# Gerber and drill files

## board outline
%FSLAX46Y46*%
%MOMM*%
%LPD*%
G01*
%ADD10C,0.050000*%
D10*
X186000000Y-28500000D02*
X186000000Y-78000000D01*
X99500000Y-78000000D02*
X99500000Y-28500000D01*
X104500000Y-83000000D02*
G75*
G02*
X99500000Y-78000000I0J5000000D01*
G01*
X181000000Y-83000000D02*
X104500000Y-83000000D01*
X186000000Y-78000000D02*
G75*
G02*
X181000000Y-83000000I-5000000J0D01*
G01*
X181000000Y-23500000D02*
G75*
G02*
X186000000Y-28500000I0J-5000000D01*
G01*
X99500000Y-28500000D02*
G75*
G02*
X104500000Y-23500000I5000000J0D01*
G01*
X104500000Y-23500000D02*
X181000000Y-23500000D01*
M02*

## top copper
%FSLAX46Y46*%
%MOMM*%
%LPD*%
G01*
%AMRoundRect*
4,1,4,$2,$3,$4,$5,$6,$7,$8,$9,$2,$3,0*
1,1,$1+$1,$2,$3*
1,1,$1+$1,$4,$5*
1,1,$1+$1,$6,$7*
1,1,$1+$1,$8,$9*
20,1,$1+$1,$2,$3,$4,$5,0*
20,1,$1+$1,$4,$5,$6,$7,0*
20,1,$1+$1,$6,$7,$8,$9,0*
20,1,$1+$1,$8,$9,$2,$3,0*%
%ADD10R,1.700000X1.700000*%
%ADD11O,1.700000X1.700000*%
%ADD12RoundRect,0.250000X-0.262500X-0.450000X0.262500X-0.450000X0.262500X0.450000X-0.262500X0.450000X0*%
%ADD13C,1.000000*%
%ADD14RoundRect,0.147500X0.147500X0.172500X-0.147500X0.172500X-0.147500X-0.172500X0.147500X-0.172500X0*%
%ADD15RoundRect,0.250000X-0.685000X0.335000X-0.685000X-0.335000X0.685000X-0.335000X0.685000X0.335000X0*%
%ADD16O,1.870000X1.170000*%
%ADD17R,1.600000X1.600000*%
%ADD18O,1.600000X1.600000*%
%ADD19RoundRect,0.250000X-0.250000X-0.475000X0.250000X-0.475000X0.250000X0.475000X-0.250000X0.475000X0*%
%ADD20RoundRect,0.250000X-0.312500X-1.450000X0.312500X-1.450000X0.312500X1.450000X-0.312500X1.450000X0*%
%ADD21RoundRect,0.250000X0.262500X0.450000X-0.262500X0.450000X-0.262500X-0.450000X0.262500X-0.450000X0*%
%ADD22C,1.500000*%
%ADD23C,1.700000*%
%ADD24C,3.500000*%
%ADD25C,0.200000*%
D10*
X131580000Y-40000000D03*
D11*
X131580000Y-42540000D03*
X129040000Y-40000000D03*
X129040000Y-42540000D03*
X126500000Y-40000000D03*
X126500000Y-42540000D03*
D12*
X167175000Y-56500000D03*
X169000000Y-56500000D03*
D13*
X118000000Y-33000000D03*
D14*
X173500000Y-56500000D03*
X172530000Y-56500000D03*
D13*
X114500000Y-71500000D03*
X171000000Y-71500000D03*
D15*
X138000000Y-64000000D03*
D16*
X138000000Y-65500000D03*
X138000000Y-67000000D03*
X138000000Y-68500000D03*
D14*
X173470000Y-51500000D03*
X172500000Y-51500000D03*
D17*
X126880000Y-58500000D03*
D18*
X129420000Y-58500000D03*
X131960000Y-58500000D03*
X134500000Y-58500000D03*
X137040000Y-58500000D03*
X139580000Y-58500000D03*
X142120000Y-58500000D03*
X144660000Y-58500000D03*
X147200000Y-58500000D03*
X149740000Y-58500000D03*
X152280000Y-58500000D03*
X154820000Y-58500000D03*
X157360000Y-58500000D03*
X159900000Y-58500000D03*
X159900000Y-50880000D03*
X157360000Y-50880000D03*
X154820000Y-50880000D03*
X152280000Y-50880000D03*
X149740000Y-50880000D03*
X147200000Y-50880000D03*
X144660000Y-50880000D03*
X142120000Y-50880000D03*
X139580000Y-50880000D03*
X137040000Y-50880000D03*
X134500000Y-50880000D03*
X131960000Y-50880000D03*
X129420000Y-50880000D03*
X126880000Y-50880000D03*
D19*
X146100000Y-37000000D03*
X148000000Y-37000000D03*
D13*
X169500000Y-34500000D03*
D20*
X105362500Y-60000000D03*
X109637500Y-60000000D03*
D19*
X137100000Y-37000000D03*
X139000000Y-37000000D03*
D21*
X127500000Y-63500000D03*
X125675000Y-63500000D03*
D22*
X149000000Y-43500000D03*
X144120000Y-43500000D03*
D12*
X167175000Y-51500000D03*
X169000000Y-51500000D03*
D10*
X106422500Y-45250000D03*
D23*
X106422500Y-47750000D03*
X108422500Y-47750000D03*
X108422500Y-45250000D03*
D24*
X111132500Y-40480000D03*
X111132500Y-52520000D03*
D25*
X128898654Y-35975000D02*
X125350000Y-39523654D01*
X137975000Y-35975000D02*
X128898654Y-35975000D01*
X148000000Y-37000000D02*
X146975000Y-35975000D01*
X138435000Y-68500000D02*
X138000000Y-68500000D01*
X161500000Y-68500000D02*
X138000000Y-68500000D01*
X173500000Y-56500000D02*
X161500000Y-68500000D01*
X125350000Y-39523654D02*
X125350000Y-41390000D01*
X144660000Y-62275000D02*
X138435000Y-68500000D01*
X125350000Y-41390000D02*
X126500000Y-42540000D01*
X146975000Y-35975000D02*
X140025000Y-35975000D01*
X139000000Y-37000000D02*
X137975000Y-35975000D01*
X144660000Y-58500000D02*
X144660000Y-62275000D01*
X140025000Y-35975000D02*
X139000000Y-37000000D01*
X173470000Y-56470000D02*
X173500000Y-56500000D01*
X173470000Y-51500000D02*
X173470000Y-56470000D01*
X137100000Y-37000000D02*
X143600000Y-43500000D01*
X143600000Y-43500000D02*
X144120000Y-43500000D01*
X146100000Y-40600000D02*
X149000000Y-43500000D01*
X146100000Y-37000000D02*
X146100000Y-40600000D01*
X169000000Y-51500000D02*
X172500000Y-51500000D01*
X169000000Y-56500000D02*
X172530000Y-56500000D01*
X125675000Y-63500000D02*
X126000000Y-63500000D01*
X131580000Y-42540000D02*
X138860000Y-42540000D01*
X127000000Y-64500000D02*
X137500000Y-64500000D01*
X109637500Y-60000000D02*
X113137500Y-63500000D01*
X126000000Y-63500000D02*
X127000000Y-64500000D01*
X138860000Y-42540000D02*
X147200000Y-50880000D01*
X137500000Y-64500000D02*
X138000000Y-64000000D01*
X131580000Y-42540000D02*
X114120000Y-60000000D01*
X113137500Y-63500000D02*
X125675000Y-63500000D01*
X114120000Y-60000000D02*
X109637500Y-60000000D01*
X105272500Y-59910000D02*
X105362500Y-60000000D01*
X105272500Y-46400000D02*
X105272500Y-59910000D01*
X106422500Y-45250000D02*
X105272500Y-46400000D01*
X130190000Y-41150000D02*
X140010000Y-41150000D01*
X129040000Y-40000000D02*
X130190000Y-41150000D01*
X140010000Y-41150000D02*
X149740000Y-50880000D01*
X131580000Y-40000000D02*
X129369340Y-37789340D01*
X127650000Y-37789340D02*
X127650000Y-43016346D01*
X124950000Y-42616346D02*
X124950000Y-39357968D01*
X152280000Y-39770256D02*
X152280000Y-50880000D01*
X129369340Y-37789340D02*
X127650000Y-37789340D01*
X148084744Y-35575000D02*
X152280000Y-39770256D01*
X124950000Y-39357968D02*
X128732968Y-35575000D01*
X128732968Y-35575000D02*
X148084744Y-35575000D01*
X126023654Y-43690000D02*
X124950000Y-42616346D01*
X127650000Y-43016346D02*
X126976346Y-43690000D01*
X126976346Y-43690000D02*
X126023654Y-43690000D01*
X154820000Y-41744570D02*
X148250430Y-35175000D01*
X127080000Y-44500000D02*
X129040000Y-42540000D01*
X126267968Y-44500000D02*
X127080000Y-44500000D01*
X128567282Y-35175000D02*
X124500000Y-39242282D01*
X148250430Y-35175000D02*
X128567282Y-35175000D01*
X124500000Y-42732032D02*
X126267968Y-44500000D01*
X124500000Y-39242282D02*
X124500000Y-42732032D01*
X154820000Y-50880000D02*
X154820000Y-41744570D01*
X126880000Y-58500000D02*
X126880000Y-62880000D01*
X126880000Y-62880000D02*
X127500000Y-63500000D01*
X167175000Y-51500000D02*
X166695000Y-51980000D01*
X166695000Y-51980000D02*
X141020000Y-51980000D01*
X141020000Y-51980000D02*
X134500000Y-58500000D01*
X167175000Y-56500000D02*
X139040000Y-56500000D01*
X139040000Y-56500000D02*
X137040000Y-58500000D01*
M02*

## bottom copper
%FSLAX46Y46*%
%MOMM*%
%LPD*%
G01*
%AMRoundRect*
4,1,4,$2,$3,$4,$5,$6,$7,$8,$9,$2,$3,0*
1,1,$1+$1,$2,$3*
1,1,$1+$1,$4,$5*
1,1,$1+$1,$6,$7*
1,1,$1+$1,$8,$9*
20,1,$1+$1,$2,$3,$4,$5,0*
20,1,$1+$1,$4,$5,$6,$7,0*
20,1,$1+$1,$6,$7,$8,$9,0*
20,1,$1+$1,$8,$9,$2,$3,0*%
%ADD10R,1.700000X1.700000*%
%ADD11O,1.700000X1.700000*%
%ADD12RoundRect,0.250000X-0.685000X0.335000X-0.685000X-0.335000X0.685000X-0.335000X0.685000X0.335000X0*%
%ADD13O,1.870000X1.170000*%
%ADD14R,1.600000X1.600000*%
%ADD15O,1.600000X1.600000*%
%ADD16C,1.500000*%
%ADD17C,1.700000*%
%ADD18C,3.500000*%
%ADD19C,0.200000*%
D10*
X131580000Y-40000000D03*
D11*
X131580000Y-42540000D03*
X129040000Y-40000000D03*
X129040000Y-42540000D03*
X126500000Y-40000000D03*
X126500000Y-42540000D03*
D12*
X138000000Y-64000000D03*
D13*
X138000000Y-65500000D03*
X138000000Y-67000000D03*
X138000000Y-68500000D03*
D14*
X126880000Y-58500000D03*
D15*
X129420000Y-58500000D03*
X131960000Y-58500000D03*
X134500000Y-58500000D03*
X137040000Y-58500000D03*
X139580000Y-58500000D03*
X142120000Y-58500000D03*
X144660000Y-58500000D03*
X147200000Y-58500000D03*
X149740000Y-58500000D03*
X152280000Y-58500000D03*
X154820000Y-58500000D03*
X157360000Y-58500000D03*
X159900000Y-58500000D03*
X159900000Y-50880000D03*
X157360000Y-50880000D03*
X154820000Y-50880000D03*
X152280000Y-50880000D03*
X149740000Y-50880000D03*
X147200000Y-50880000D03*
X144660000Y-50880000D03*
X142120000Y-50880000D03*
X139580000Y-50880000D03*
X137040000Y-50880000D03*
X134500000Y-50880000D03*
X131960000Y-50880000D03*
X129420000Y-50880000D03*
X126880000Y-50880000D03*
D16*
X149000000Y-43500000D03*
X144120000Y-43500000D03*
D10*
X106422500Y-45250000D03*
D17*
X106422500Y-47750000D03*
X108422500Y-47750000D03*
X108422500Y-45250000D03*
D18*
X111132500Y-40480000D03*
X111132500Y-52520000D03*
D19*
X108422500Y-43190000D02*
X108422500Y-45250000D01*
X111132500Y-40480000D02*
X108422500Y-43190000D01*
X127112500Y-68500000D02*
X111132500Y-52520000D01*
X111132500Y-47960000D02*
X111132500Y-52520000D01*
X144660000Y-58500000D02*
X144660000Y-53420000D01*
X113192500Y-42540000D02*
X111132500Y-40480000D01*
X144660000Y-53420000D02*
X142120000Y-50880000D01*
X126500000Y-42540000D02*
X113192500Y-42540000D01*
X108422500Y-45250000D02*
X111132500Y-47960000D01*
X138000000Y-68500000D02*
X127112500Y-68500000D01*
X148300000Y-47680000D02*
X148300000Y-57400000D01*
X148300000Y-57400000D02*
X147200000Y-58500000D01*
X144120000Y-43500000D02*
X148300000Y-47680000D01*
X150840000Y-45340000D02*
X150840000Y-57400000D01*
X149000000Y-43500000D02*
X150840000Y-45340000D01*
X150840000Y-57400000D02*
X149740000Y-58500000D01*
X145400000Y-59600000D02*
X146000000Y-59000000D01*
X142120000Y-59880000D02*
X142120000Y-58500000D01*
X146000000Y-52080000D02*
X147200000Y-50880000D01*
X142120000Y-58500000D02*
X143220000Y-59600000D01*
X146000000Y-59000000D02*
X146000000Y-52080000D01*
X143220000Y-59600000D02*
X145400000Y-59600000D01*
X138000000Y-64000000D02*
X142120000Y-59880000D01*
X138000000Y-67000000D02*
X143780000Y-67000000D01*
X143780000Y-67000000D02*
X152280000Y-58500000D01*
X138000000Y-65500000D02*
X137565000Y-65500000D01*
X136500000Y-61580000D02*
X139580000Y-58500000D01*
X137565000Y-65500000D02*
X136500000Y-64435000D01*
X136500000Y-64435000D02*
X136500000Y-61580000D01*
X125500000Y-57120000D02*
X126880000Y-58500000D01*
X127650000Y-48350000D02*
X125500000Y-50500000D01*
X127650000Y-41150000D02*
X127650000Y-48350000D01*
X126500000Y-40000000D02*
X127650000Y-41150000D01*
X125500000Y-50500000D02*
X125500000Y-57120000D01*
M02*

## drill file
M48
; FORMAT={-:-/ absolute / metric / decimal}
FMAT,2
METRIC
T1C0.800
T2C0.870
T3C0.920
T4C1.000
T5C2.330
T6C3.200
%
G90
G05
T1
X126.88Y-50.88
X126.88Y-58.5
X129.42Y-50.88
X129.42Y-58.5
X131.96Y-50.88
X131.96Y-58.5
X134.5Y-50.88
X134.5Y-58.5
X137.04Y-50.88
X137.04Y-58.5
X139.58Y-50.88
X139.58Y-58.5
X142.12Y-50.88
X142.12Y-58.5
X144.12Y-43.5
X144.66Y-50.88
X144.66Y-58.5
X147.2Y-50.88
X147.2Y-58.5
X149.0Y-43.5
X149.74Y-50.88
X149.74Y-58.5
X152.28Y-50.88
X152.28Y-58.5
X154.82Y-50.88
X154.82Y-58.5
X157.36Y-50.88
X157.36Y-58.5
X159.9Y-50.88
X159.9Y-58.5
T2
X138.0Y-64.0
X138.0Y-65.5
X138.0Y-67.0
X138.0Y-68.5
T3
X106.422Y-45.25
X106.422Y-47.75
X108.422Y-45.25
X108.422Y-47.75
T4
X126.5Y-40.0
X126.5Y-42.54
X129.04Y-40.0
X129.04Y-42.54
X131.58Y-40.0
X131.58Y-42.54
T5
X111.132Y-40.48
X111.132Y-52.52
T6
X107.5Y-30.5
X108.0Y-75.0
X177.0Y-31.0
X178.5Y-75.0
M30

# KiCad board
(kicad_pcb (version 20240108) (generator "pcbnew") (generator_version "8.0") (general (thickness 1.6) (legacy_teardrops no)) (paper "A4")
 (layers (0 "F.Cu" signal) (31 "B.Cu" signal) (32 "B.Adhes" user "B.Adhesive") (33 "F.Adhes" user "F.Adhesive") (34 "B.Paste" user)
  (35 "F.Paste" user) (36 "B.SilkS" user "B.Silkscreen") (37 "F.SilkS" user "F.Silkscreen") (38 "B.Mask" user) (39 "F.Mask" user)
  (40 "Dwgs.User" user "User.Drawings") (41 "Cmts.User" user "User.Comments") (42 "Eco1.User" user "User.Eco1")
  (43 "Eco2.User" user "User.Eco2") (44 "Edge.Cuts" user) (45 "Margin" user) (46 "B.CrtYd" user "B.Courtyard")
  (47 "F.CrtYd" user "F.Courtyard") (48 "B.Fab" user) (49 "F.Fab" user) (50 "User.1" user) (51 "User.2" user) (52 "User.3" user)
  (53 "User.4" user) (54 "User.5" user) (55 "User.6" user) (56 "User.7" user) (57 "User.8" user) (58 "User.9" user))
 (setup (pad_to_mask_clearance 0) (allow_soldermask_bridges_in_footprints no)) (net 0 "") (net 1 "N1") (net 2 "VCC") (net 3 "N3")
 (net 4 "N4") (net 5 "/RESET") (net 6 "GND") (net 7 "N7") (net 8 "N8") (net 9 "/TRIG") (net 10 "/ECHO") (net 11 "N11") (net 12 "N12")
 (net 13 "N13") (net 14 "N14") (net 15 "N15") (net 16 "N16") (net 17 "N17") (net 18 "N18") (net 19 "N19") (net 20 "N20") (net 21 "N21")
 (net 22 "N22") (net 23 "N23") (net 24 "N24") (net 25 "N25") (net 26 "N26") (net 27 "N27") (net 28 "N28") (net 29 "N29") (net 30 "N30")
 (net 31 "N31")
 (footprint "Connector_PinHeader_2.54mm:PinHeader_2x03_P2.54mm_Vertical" (layer "F.Cu") (at 131.58 40 -90)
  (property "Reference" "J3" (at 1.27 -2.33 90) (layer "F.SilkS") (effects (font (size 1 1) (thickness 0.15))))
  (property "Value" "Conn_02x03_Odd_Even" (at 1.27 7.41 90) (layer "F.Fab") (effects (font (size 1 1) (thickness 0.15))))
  (pad "1" thru_hole rect (at 0 0 270) (size 1.7 1.7) (drill 1) (layers "*.Cu" "*.Mask") (remove_unused_layers no) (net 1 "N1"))
  (pad "2" thru_hole oval (at 2.54 0 270) (size 1.7 1.7) (drill 1) (layers "*.Cu" "*.Mask") (remove_unused_layers no) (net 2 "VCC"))
  (pad "3" thru_hole oval (at 0 2.54 270) (size 1.7 1.7) (drill 1) (layers "*.Cu" "*.Mask") (remove_unused_layers no) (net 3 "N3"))
  (pad "4" thru_hole oval (at 2.54 2.54 270) (size 1.7 1.7) (drill 1) (layers "*.Cu" "*.Mask") (remove_unused_layers no) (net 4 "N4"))
  (pad "5" thru_hole oval (at 0 5.08 270) (size 1.7 1.7) (drill 1) (layers "*.Cu" "*.Mask") (remove_unused_layers no) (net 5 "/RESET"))
  (pad "6" thru_hole oval (at 2.54 5.08 270) (size 1.7 1.7) (drill 1) (layers "*.Cu" "*.Mask") (remove_unused_layers no) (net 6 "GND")))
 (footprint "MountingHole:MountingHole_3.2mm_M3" (layer "F.Cu") (at 108 75)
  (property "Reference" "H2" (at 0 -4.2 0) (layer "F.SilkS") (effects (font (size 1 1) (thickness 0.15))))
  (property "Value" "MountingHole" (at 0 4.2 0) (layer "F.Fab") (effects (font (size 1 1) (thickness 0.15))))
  (pad "" np_thru_hole circle (at 0 0) (size 3.2 3.2) (drill 3.2) (layers "*.Cu" "*.Mask")))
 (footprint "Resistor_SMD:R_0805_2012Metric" (layer "F.Cu") (at 168.0875 56.5)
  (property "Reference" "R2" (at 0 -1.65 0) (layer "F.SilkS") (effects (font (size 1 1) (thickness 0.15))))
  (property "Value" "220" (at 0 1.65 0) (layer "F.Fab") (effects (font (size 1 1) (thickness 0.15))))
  (pad "1" smd roundrect (at -0.9125 0) (size 1.025 1.4) (layers "F.Cu" "F.Paste" "F.Mask") (roundrect_rratio 0.243902) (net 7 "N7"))
  (pad "2" smd roundrect (at 0.9125 0) (size 1.025 1.4) (layers "F.Cu" "F.Paste" "F.Mask") (roundrect_rratio 0.243902) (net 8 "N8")))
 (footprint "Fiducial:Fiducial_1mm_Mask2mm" (layer "F.Cu") (at 118 33)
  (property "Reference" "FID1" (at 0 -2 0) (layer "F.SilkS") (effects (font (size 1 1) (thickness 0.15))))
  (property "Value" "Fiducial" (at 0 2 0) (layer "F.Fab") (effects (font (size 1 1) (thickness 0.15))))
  (pad "" smd circle (at 0 0) (size 1 1) (layers "F.Cu" "F.Mask") (solder_mask_margin 0.5) (clearance 0.5)))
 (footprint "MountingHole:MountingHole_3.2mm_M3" (layer "F.Cu") (at 177 31)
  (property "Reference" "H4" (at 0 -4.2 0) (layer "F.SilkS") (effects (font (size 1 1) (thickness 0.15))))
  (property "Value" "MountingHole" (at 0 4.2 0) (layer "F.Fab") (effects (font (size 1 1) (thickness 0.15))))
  (pad "" np_thru_hole circle (at 0 0) (size 3.2 3.2) (drill 3.2) (layers "*.Cu" "*.Mask")))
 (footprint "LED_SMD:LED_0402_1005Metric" (layer "F.Cu") (at 173.015 56.5 180)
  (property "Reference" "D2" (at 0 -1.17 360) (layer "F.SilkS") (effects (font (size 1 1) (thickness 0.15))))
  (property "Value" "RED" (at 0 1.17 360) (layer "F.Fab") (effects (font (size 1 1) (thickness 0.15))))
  (pad "1" smd roundrect (at -0.485 0 180) (size 0.59 0.64) (layers "F.Cu" "F.Paste" "F.Mask") (roundrect_rratio 0.25) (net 6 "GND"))
  (pad "2" smd roundrect (at 0.485 0 180) (size 0.59 0.64) (layers "F.Cu" "F.Paste" "F.Mask") (roundrect_rratio 0.25) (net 8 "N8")))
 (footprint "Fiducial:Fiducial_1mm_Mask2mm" (layer "F.Cu") (at 114.5 71.5)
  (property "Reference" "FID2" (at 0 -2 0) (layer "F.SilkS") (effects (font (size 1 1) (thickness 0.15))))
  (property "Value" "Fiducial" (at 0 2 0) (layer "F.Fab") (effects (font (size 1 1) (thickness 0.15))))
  (pad "" smd circle (at 0 0) (size 1 1) (layers "F.Cu" "F.Mask") (solder_mask_margin 0.5) (clearance 0.5)))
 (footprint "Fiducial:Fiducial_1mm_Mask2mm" (layer "F.Cu") (at 171 71.5)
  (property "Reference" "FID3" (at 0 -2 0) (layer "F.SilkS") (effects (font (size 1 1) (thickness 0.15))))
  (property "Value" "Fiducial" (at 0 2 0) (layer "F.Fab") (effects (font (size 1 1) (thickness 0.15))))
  (pad "" smd circle (at 0 0) (size 1 1) (layers "F.Cu" "F.Mask") (solder_mask_margin 0.5) (clearance 0.5)))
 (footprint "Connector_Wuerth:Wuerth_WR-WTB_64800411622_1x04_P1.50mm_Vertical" (layer "F.Cu") (at 138 64 -90)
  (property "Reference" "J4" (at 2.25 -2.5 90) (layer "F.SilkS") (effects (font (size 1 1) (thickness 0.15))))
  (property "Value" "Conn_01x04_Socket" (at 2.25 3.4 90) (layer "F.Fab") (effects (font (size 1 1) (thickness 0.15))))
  (pad "1" thru_hole roundrect (at 0 0 270) (size 1.17 1.87) (drill 0.87) (layers "*.Cu" "*.Mask") (remove_unused_layers no)
   (roundrect_rratio 0.213675) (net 2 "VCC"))
  (pad "2" thru_hole oval (at 1.5 0 270) (size 1.17 1.87) (drill 0.87) (layers "*.Cu" "*.Mask") (remove_unused_layers no) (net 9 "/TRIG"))
  (pad "3" thru_hole oval (at 3 0 270) (size 1.17 1.87) (drill 0.87) (layers "*.Cu" "*.Mask") (remove_unused_layers no) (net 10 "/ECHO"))
  (pad "4" thru_hole oval (at 4.5 0 270) (size 1.17 1.87) (drill 0.87) (layers "*.Cu" "*.Mask") (remove_unused_layers no) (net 6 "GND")))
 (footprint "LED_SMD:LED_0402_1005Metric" (layer "F.Cu") (at 172.985 51.5 180)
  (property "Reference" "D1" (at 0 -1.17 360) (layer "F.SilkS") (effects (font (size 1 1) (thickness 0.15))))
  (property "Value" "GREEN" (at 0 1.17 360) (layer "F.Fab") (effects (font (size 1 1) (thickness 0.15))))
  (pad "1" smd roundrect (at -0.485 0 180) (size 0.59 0.64) (layers "F.Cu" "F.Paste" "F.Mask") (roundrect_rratio 0.25) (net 6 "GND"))
  (pad "2" smd roundrect (at 0.485 0 180) (size 0.59 0.64) (layers "F.Cu" "F.Paste" "F.Mask") (roundrect_rratio 0.25) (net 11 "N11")))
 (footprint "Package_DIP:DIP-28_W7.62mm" (layer "F.Cu") (at 126.88 58.5 90)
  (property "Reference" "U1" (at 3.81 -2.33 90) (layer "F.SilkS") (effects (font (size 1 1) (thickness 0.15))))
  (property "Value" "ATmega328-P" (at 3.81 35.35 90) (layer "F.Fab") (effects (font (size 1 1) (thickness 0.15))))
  (pad "1" thru_hole rect (at 0 0 90) (size 1.6 1.6) (drill 0.8) (layers "*.Cu" "*.Mask") (remove_unused_layers no) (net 5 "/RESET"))
  (pad "2" thru_hole oval (at 0 2.54 90) (size 1.6 1.6) (drill 0.8) (layers "*.Cu" "*.Mask") (remove_unused_layers no) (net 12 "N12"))
  (pad "3" thru_hole oval (at 0 5.08 90) (size 1.6 1.6) (drill 0.8) (layers "*.Cu" "*.Mask") (remove_unused_layers no) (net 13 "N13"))
  (pad "4" thru_hole oval (at 0 7.62 90) (size 1.6 1.6) (drill 0.8) (layers "*.Cu" "*.Mask") (remove_unused_layers no) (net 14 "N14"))
  (pad "5" thru_hole oval (at 0 10.16 90) (size 1.6 1.6) (drill 0.8) (layers "*.Cu" "*.Mask") (remove_unused_layers no) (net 7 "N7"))
  (pad "6" thru_hole oval (at 0 12.7 90) (size 1.6 1.6) (drill 0.8) (layers "*.Cu" "*.Mask") (remove_unused_layers no) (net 9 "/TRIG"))
  (pad "7" thru_hole oval (at 0 15.24 90) (size 1.6 1.6) (drill 0.8) (layers "*.Cu" "*.Mask") (remove_unused_layers no) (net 2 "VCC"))
  (pad "8" thru_hole oval (at 0 17.78 90) (size 1.6 1.6) (drill 0.8) (layers "*.Cu" "*.Mask") (remove_unused_layers no) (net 6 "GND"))
  (pad "9" thru_hole oval (at 0 20.32 90) (size 1.6 1.6) (drill 0.8) (layers "*.Cu" "*.Mask") (remove_unused_layers no) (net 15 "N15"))
  (pad "10" thru_hole oval (at 0 22.86 90) (size 1.6 1.6) (drill 0.8) (layers "*.Cu" "*.Mask") (remove_unused_layers no) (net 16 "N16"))
  (pad "11" thru_hole oval (at 0 25.4 90) (size 1.6 1.6) (drill 0.8) (layers "*.Cu" "*.Mask") (remove_unused_layers no) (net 10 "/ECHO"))
  (pad "12" thru_hole oval (at 0 27.94 90) (size 1.6 1.6) (drill 0.8) (layers "*.Cu" "*.Mask") (remove_unused_layers no) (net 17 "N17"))
  (pad "13" thru_hole oval (at 0 30.48 90) (size 1.6 1.6) (drill 0.8) (layers "*.Cu" "*.Mask") (remove_unused_layers no) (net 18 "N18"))
  (pad "14" thru_hole oval (at 0 33.02 90) (size 1.6 1.6) (drill 0.8) (layers "*.Cu" "*.Mask") (remove_unused_layers no) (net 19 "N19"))
  (pad "15" thru_hole oval (at 7.62 33.02 90) (size 1.6 1.6) (drill 0.8) (layers "*.Cu" "*.Mask") (remove_unused_layers no) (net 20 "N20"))
  (pad "16" thru_hole oval (at 7.62 30.48 90) (size 1.6 1.6) (drill 0.8) (layers "*.Cu" "*.Mask") (remove_unused_layers no) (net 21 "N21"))
  (pad "17" thru_hole oval (at 7.62 27.94 90) (size 1.6 1.6) (drill 0.8) (layers "*.Cu" "*.Mask") (remove_unused_layers no) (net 4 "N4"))
  (pad "18" thru_hole oval (at 7.62 25.4 90) (size 1.6 1.6) (drill 0.8) (layers "*.Cu" "*.Mask") (remove_unused_layers no) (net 1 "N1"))
  (pad "19" thru_hole oval (at 7.62 22.86 90) (size 1.6 1.6) (drill 0.8) (layers "*.Cu" "*.Mask") (remove_unused_layers no) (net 3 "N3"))
  (pad "20" thru_hole oval (at 7.62 20.32 90) (size 1.6 1.6) (drill 0.8) (layers "*.Cu" "*.Mask") (remove_unused_layers no) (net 2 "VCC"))
  (pad "21" thru_hole oval (at 7.62 17.78 90) (size 1.6 1.6) (drill 0.8) (layers "*.Cu" "*.Mask") (remove_unused_layers no) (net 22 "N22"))
  (pad "22" thru_hole oval (at 7.62 15.24 90) (size 1.6 1.6) (drill 0.8) (layers "*.Cu" "*.Mask") (remove_unused_layers no) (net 6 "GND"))
  (pad "23" thru_hole oval (at 7.62 12.7 90) (size 1.6 1.6) (drill 0.8) (layers "*.Cu" "*.Mask") (remove_unused_layers no) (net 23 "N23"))
  (pad "24" thru_hole oval (at 7.62 10.16 90) (size 1.6 1.6) (drill 0.8) (layers "*.Cu" "*.Mask") (remove_unused_layers no) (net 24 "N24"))
  (pad "25" thru_hole oval (at 7.62 7.62 90) (size 1.6 1.6) (drill 0.8) (layers "*.Cu" "*.Mask") (remove_unused_layers no) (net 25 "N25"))
  (pad "26" thru_hole oval (at 7.62 5.08 90) (size 1.6 1.6) (drill 0.8) (layers "*.Cu" "*.Mask") (remove_unused_layers no) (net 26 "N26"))
  (pad "27" thru_hole oval (at 7.62 2.54 90) (size 1.6 1.6) (drill 0.8) (layers "*.Cu" "*.Mask") (remove_unused_layers no) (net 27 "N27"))
  (pad "28" thru_hole oval (at 7.62 0 90) (size 1.6 1.6) (drill 0.8) (layers "*.Cu" "*.Mask") (remove_unused_layers no) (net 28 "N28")))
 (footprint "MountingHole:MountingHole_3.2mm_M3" (layer "F.Cu") (at 178.5 75)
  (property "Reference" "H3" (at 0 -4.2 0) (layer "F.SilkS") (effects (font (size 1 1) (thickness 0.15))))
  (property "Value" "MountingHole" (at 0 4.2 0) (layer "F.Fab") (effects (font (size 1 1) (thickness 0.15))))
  (pad "" np_thru_hole circle (at 0 0) (size 3.2 3.2) (drill 3.2) (layers "*.Cu" "*.Mask")))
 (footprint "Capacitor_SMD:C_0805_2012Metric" (layer "F.Cu") (at 147.05 37)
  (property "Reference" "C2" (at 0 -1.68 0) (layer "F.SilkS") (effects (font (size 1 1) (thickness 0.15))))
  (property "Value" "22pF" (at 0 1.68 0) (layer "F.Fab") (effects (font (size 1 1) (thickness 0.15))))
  (pad "1" smd roundrect (at -0.95 0) (size 1 1.45) (layers "F.Cu" "F.Paste" "F.Mask") (roundrect_rratio 0.25) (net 16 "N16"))
  (pad "2" smd roundrect (at 0.95 0) (size 1 1.45) (layers "F.Cu" "F.Paste" "F.Mask") (roundrect_rratio 0.25) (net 6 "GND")))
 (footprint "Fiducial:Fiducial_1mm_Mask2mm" (layer "F.Cu") (at 169.5 34.5)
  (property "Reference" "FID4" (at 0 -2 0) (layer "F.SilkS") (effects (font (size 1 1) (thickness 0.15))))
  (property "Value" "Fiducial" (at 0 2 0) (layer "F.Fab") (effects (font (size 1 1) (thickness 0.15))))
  (pad "" smd circle (at 0 0) (size 1 1) (layers "F.Cu" "F.Mask") (solder_mask_margin 0.5) (clearance 0.5)))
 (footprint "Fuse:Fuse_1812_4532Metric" (layer "F.Cu") (at 107.5 60)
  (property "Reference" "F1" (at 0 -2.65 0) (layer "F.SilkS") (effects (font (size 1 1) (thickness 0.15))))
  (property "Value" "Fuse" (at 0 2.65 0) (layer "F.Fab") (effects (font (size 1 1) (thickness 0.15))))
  (pad "1" smd roundrect (at -2.1375 0) (size 1.125 3.4) (layers "F.Cu" "F.Paste" "F.Mask") (roundrect_rratio 0.222222) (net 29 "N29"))
  (pad "2" smd roundrect (at 2.1375 0) (size 1.125 3.4) (layers "F.Cu" "F.Paste" "F.Mask") (roundrect_rratio 0.222222) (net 2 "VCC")))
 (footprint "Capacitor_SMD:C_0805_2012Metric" (layer "F.Cu") (at 138.05 37)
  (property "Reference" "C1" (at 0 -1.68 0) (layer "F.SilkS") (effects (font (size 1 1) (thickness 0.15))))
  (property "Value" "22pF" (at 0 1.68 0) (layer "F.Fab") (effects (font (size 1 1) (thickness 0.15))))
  (pad "1" smd roundrect (at -0.95 0) (size 1 1.45) (layers "F.Cu" "F.Paste" "F.Mask") (roundrect_rratio 0.25) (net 15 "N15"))
  (pad "2" smd roundrect (at 0.95 0) (size 1 1.45) (layers "F.Cu" "F.Paste" "F.Mask") (roundrect_rratio 0.25) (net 6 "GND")))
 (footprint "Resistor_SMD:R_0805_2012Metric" (layer "F.Cu") (at 126.5875 63.5 180)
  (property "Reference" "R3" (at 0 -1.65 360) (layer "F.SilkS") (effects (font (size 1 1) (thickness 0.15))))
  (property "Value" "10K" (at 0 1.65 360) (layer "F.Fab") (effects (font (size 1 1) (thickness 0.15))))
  (pad "1" smd roundrect (at -0.9125 0 180) (size 1.025 1.4) (layers "F.Cu" "F.Paste" "F.Mask") (roundrect_rratio 0.243902) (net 5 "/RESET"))
  (pad "2" smd roundrect (at 0.9125 0 180) (size 1.025 1.4) (layers "F.Cu" "F.Paste" "F.Mask") (roundrect_rratio 0.243902) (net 2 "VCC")))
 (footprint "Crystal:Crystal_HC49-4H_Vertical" (layer "F.Cu") (at 149 43.5 180)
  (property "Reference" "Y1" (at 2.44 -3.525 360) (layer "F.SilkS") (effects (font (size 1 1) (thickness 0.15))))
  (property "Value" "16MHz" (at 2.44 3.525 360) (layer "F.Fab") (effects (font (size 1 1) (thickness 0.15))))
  (pad "1" thru_hole circle (at 0 0 180) (size 1.5 1.5) (drill 0.8) (layers "*.Cu" "*.Mask") (remove_unused_layers no) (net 16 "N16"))
  (pad "2" thru_hole circle (at 4.88 0 180) (size 1.5 1.5) (drill 0.8) (layers "*.Cu" "*.Mask") (remove_unused_layers no) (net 15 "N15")))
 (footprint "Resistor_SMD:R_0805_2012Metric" (layer "F.Cu") (at 168.0875 51.5)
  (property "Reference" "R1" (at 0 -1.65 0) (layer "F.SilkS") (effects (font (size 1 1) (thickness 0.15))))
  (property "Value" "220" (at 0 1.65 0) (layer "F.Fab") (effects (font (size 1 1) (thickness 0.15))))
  (pad "1" smd roundrect (at -0.9125 0) (size 1.025 1.4) (layers "F.Cu" "F.Paste" "F.Mask") (roundrect_rratio 0.243902) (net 14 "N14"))
  (pad "2" smd roundrect (at 0.9125 0) (size 1.025 1.4) (layers "F.Cu" "F.Paste" "F.Mask") (roundrect_rratio 0.243902) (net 11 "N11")))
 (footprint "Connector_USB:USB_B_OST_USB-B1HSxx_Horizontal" (layer "F.Cu") (at 106.4225 45.25)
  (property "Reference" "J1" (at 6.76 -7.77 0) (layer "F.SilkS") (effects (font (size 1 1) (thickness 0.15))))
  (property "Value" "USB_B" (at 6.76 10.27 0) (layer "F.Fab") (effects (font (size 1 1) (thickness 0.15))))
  (pad "1" thru_hole rect (at 0 0) (size 1.7 1.7) (drill 0.92) (layers "*.Cu" "*.Mask") (remove_unused_layers no) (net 29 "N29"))
  (pad "2" thru_hole circle (at 0 2.5) (size 1.7 1.7) (drill 0.92) (layers "*.Cu" "*.Mask") (remove_unused_layers no) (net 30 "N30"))
  (pad "3" thru_hole circle (at 2 2.5) (size 1.7 1.7) (drill 0.92) (layers "*.Cu" "*.Mask") (remove_unused_layers no) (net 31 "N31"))
  (pad "4" thru_hole circle (at 2 0) (size 1.7 1.7) (drill 0.92) (layers "*.Cu" "*.Mask") (remove_unused_layers no) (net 6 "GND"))
  (pad "5" thru_hole circle (at 4.71 -4.77) (size 3.5 3.5) (drill 2.33) (layers "*.Cu" "*.Mask") (remove_unused_layers no) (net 6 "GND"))
  (pad "5" thru_hole circle (at 4.71 7.27) (size 3.5 3.5) (drill 2.33) (layers "*.Cu" "*.Mask") (remove_unused_layers no) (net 6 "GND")))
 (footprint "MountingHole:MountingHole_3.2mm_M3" (layer "F.Cu") (at 107.5 30.5)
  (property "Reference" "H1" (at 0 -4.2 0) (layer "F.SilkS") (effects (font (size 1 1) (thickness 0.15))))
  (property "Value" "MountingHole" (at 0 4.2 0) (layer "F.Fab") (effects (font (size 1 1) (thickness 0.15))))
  (pad "" np_thru_hole circle (at 0 0) (size 3.2 3.2) (drill 3.2) (layers "*.Cu" "*.Mask")))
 (gr_line (start 186 28.5) (end 186 78) (stroke (width 0.05) (type default)) (layer "Edge.Cuts"))
 (gr_line (start 99.5 78) (end 99.5 28.5) (stroke (width 0.05) (type default)) (layer "Edge.Cuts"))
 (gr_arc (start 104.5 83) (mid 100.964466 81.535534) (end 99.5 78) (stroke (width 0.05) (type default)) (layer "Edge.Cuts"))
 (gr_line (start 181 83) (end 104.5 83) (stroke (width 0.05) (type default)) (layer "Edge.Cuts"))
 (gr_arc (start 186 78) (mid 184.535534 81.535534) (end 181 83) (stroke (width 0.05) (type default)) (layer "Edge.Cuts"))
 (gr_arc (start 181 23.5) (mid 184.535534 24.964466) (end 186 28.5) (stroke (width 0.05) (type default)) (layer "Edge.Cuts"))
 (gr_arc (start 99.5 28.5) (mid 100.964466 24.964466) (end 104.5 23.5) (stroke (width 0.05) (type default)) (layer "Edge.Cuts"))
 (gr_line (start 104.5 23.5) (end 181 23.5) (stroke (width 0.05) (type default)) (layer "Edge.Cuts"))
 (segment (start 128.898654 35.975) (end 125.35 39.523654) (width 0.2) (layer "F.Cu") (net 6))
 (segment (start 137.975 35.975) (end 128.898654 35.975) (width 0.2) (layer "F.Cu") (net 6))
 (segment (start 148 37) (end 146.975 35.975) (width 0.2) (layer "F.Cu") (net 6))
 (segment (start 138.435 68.5) (end 138 68.5) (width 0.2) (layer "F.Cu") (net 6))
 (segment (start 161.5 68.5) (end 138 68.5) (width 0.2) (layer "F.Cu") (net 6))
 (segment (start 173.5 56.5) (end 161.5 68.5) (width 0.2) (layer "F.Cu") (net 6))
 (segment (start 125.35 39.523654) (end 125.35 41.39) (width 0.2) (layer "F.Cu") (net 6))
 (segment (start 144.66 62.275) (end 138.435 68.5) (width 0.2) (layer "F.Cu") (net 6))
 (segment (start 125.35 41.39) (end 126.5 42.54) (width 0.2) (layer "F.Cu") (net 6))
 (segment (start 146.975 35.975) (end 140.025 35.975) (width 0.2) (layer "F.Cu") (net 6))
 (segment (start 139 37) (end 137.975 35.975) (width 0.2) (layer "F.Cu") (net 6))
 (segment (start 144.66 58.5) (end 144.66 62.275) (width 0.2) (layer "F.Cu") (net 6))
 (segment (start 140.025 35.975) (end 139 37) (width 0.2) (layer "F.Cu") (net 6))
 (segment (start 173.47 56.47) (end 173.5 56.5) (width 0.2) (layer "F.Cu") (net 6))
 (segment (start 173.47 51.5) (end 173.47 56.47) (width 0.2) (layer "F.Cu") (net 6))
 (segment (start 108.4225 43.19) (end 108.4225 45.25) (width 0.2) (layer "B.Cu") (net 6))
 (segment (start 111.1325 40.48) (end 108.4225 43.19) (width 0.2) (layer "B.Cu") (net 6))
 (segment (start 127.1125 68.5) (end 111.1325 52.52) (width 0.2) (layer "B.Cu") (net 6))
 (segment (start 111.1325 47.96) (end 111.1325 52.52) (width 0.2) (layer "B.Cu") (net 6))
 (segment (start 144.66 58.5) (end 144.66 53.42) (width 0.2) (layer "B.Cu") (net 6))
 (segment (start 113.1925 42.54) (end 111.1325 40.48) (width 0.2) (layer "B.Cu") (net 6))
 (segment (start 144.66 53.42) (end 142.12 50.88) (width 0.2) (layer "B.Cu") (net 6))
 (segment (start 126.5 42.54) (end 113.1925 42.54) (width 0.2) (layer "B.Cu") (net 6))
 (segment (start 108.4225 45.25) (end 111.1325 47.96) (width 0.2) (layer "B.Cu") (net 6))
 (segment (start 138 68.5) (end 127.1125 68.5) (width 0.2) (layer "B.Cu") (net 6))
 (segment (start 137.1 37) (end 143.6 43.5) (width 0.2) (layer "F.Cu") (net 15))
 (segment (start 143.6 43.5) (end 144.12 43.5) (width 0.2) (layer "F.Cu") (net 15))
 (segment (start 148.3 47.68) (end 148.3 57.4) (width 0.2) (layer "B.Cu") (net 15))
 (segment (start 148.3 57.4) (end 147.2 58.5) (width 0.2) (layer "B.Cu") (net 15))
 (segment (start 144.12 43.5) (end 148.3 47.68) (width 0.2) (layer "B.Cu") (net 15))
 (segment (start 146.1 40.6) (end 149 43.5) (width 0.2) (layer "F.Cu") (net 16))
 (segment (start 146.1 37) (end 146.1 40.6) (width 0.2) (layer "F.Cu") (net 16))
 (segment (start 150.84 45.34) (end 150.84 57.4) (width 0.2) (layer "B.Cu") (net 16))
 (segment (start 149 43.5) (end 150.84 45.34) (width 0.2) (layer "B.Cu") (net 16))
 (segment (start 150.84 57.4) (end 149.74 58.5) (width 0.2) (layer "B.Cu") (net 16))
 (segment (start 169 51.5) (end 172.5 51.5) (width 0.2) (layer "F.Cu") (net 11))
 (segment (start 169 56.5) (end 172.53 56.5) (width 0.2) (layer "F.Cu") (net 8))
 (segment (start 125.675 63.5) (end 126 63.5) (width 0.2) (layer "F.Cu") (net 2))
 (segment (start 131.58 42.54) (end 138.86 42.54) (width 0.2) (layer "F.Cu") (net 2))
 (segment (start 127 64.5) (end 137.5 64.5) (width 0.2) (layer "F.Cu") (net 2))
 (segment (start 109.6375 60) (end 113.1375 63.5) (width 0.2) (layer "F.Cu") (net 2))
 (segment (start 126 63.5) (end 127 64.5) (width 0.2) (layer "F.Cu") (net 2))
 (segment (start 138.86 42.54) (end 147.2 50.88) (width 0.2) (layer "F.Cu") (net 2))
 (segment (start 137.5 64.5) (end 138 64) (width 0.2) (layer "F.Cu") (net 2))
 (segment (start 131.58 42.54) (end 114.12 60) (width 0.2) (layer "F.Cu") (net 2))
 (segment (start 113.1375 63.5) (end 125.675 63.5) (width 0.2) (layer "F.Cu") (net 2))
 (segment (start 114.12 60) (end 109.6375 60) (width 0.2) (layer "F.Cu") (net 2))
 (segment (start 145.4 59.6) (end 146 59) (width 0.2) (layer "B.Cu") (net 2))
 (segment (start 142.12 59.88) (end 142.12 58.5) (width 0.2) (layer "B.Cu") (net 2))
 (segment (start 146 52.08) (end 147.2 50.88) (width 0.2) (layer "B.Cu") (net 2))
 (segment (start 142.12 58.5) (end 143.22 59.6) (width 0.2) (layer "B.Cu") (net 2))
 (segment (start 146 59) (end 146 52.08) (width 0.2) (layer "B.Cu") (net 2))
 (segment (start 143.22 59.6) (end 145.4 59.6) (width 0.2) (layer "B.Cu") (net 2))
 (segment (start 138 64) (end 142.12 59.88) (width 0.2) (layer "B.Cu") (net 2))
 (segment (start 105.2725 59.91) (end 105.3625 60) (width 0.2) (layer "F.Cu") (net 29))
 (segment (start 105.2725 46.4) (end 105.2725 59.91) (width 0.2) (layer "F.Cu") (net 29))
 (segment (start 106.4225 45.25) (end 105.2725 46.4) (width 0.2) (layer "F.Cu") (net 29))
 (segment (start 138 67) (end 143.78 67) (width 0.2) (layer "B.Cu") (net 10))
 (segment (start 143.78 67) (end 152.28 58.5) (width 0.2) (layer "B.Cu") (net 10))
 (segment (start 138 65.5) (end 137.565 65.5) (width 0.2) (layer "B.Cu") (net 9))
 (segment (start 136.5 61.58) (end 139.58 58.5) (width 0.2) (layer "B.Cu") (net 9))
 (segment (start 137.565 65.5) (end 136.5 64.435) (width 0.2) (layer "B.Cu") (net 9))
 (segment (start 136.5 64.435) (end 136.5 61.58) (width 0.2) (layer "B.Cu") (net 9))
 (segment (start 130.19 41.15) (end 140.01 41.15) (width 0.2) (layer "F.Cu") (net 3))
 (segment (start 129.04 40) (end 130.19 41.15) (width 0.2) (layer "F.Cu") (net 3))
 (segment (start 140.01 41.15) (end 149.74 50.88) (width 0.2) (layer "F.Cu") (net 3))
 (segment (start 131.58 40) (end 129.36934 37.78934) (width 0.2) (layer "F.Cu") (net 1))
 (segment (start 127.65 37.78934) (end 127.65 43.016346) (width 0.2) (layer "F.Cu") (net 1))
 (segment (start 124.95 42.616346) (end 124.95 39.357968) (width 0.2) (layer "F.Cu") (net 1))
 (segment (start 152.28 39.770256) (end 152.28 50.88) (width 0.2) (layer "F.Cu") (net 1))
 (segment (start 129.36934 37.78934) (end 127.65 37.78934) (width 0.2) (layer "F.Cu") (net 1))
 (segment (start 148.084744 35.575) (end 152.28 39.770256) (width 0.2) (layer "F.Cu") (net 1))
 (segment (start 124.95 39.357968) (end 128.732968 35.575) (width 0.2) (layer "F.Cu") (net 1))
 (segment (start 128.732968 35.575) (end 148.084744 35.575) (width 0.2) (layer "F.Cu") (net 1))
 (segment (start 126.023654 43.69) (end 124.95 42.616346) (width 0.2) (layer "F.Cu") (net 1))
 (segment (start 127.65 43.016346) (end 126.976346 43.69) (width 0.2) (layer "F.Cu") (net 1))
 (segment (start 126.976346 43.69) (end 126.023654 43.69) (width 0.2) (layer "F.Cu") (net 1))
 (segment (start 154.82 41.74457) (end 148.25043 35.175) (width 0.2) (layer "F.Cu") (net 4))
 (segment (start 127.08 44.5) (end 129.04 42.54) (width 0.2) (layer "F.Cu") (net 4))
 (segment (start 126.267968 44.5) (end 127.08 44.5) (width 0.2) (layer "F.Cu") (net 4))
 (segment (start 128.567282 35.175) (end 124.5 39.242282) (width 0.2) (layer "F.Cu") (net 4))
 (segment (start 148.25043 35.175) (end 128.567282 35.175) (width 0.2) (layer "F.Cu") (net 4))
 (segment (start 124.5 42.732032) (end 126.267968 44.5) (width 0.2) (layer "F.Cu") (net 4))
 (segment (start 124.5 39.242282) (end 124.5 42.732032) (width 0.2) (layer "F.Cu") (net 4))
 (segment (start 154.82 50.88) (end 154.82 41.74457) (width 0.2) (layer "F.Cu") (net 4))
 (segment (start 126.88 58.5) (end 126.88 62.88) (width 0.2) (layer "F.Cu") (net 5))
 (segment (start 126.88 62.88) (end 127.5 63.5) (width 0.2) (layer "F.Cu") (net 5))
 (segment (start 125.5 57.12) (end 126.88 58.5) (width 0.2) (layer "B.Cu") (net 5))
 (segment (start 127.65 48.35) (end 125.5 50.5) (width 0.2) (layer "B.Cu") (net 5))
 (segment (start 127.65 41.15) (end 127.65 48.35) (width 0.2) (layer "B.Cu") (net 5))
 (segment (start 126.5 40) (end 127.65 41.15) (width 0.2) (layer "B.Cu") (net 5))
 (segment (start 125.5 50.5) (end 125.5 57.12) (width 0.2) (layer "B.Cu") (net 5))
 (segment (start 167.175 51.5) (end 166.695 51.98) (width 0.2) (layer "F.Cu") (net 14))
 (segment (start 166.695 51.98) (end 141.02 51.98) (width 0.2) (layer "F.Cu") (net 14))
 (segment (start 141.02 51.98) (end 134.5 58.5) (width 0.2) (layer "F.Cu") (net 14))
 (segment (start 167.175 56.5) (end 139.04 56.5) (width 0.2) (layer "F.Cu") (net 7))
 (segment (start 139.04 56.5) (end 137.04 58.5) (width 0.2) (layer "F.Cu") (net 7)))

